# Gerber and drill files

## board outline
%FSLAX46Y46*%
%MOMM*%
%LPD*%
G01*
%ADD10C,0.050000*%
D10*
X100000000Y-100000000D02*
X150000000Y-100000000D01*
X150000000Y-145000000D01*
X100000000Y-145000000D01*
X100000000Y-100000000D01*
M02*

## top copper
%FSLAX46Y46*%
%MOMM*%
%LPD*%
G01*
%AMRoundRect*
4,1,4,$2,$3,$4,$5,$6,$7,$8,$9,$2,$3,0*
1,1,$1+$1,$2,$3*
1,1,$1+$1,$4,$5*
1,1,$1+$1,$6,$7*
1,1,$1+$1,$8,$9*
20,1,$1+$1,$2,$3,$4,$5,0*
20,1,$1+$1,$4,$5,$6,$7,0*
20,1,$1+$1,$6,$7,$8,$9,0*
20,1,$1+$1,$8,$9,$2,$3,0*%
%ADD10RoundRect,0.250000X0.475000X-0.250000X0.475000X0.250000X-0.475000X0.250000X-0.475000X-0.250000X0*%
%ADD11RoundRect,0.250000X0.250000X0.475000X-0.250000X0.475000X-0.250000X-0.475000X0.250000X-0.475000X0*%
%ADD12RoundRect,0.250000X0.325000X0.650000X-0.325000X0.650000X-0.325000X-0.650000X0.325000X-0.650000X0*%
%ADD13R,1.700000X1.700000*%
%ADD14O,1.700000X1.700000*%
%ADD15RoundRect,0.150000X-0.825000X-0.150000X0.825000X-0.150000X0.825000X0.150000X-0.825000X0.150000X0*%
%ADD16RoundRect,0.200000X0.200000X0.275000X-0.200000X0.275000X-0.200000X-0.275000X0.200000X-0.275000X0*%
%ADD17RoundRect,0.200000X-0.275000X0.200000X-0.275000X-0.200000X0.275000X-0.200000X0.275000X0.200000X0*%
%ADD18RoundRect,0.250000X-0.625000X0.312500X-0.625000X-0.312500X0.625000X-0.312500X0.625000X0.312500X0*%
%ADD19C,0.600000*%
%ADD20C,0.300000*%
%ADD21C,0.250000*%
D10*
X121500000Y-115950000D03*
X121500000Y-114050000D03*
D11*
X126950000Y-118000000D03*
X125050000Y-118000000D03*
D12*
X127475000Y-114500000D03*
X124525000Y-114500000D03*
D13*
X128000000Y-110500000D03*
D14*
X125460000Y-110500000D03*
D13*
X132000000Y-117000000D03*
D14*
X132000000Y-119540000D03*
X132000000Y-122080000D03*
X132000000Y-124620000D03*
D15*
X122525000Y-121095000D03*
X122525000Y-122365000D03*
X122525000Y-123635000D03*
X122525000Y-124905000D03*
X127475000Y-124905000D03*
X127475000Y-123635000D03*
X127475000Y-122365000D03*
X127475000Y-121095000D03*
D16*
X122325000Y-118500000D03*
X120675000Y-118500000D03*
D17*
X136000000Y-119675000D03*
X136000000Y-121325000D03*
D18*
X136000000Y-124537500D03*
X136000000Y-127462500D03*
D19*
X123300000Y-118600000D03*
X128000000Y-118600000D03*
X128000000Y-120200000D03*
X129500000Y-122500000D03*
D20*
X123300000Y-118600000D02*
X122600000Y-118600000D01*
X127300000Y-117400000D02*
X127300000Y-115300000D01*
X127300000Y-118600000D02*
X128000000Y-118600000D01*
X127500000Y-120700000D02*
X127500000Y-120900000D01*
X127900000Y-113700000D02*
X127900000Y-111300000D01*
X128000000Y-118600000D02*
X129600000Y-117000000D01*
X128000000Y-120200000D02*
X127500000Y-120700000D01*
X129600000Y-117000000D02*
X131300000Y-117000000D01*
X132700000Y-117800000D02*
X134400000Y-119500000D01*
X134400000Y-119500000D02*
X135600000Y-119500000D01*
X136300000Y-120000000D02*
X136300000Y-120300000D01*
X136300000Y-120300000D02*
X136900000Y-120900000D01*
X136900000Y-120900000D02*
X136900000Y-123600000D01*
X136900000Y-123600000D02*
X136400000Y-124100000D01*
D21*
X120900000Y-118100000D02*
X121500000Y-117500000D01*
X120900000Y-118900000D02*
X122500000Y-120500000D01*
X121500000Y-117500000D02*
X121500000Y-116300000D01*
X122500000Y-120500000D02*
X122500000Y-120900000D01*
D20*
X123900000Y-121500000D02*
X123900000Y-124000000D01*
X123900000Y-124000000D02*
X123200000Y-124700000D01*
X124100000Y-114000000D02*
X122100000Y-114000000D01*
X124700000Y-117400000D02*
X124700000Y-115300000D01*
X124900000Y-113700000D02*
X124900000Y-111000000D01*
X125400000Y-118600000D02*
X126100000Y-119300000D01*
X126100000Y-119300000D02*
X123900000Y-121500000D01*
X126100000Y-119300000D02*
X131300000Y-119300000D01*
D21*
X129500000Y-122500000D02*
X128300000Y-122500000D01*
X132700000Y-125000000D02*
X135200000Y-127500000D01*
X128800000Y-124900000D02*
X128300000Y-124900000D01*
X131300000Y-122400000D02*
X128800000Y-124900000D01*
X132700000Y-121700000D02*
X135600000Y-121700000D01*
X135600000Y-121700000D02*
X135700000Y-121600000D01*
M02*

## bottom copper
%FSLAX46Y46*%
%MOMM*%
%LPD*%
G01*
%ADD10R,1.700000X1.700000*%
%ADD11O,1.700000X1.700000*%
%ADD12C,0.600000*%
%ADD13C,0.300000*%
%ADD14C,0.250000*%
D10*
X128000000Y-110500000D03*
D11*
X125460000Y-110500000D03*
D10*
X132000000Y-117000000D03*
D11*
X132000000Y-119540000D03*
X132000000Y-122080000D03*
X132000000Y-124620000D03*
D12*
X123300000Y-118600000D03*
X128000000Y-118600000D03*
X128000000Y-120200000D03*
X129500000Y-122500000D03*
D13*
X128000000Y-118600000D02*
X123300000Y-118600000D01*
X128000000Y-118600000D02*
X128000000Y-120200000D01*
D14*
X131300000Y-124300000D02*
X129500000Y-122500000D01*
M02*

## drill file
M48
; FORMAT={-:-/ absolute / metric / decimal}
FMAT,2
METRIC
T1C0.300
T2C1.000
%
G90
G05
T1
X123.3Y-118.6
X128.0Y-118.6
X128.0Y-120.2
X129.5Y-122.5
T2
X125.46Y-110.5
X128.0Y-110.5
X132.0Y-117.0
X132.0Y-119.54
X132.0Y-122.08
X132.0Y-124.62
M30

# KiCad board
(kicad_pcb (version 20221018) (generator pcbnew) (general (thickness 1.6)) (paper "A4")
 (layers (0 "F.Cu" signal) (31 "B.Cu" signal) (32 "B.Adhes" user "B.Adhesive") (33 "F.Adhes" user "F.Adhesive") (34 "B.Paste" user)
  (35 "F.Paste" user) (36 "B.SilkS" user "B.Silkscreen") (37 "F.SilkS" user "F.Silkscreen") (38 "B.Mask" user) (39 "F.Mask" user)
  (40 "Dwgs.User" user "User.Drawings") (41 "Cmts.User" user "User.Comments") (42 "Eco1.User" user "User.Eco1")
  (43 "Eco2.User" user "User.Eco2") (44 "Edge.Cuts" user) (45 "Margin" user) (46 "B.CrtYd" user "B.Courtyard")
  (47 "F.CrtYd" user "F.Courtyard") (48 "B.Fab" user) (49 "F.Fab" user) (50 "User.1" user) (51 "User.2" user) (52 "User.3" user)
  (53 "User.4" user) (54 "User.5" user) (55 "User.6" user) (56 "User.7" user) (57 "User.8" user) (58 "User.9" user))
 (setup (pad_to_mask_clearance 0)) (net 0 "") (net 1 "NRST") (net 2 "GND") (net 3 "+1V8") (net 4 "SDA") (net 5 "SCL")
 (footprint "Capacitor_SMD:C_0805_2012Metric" (layer "F.Cu") (at 121.5 115 90)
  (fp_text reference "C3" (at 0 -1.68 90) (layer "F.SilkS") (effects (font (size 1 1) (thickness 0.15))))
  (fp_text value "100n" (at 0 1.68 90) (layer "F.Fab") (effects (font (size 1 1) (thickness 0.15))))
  (pad "1" smd roundrect (at -0.95 0 90) (size 1 1.45) (layers "F.Cu" "F.Paste" "F.Mask") (roundrect_rratio 0.25) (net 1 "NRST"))
  (pad "2" smd roundrect (at 0.95 0 90) (size 1 1.45) (layers "F.Cu" "F.Paste" "F.Mask") (roundrect_rratio 0.25) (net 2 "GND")))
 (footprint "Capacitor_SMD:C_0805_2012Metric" (layer "F.Cu") (at 126 118 180)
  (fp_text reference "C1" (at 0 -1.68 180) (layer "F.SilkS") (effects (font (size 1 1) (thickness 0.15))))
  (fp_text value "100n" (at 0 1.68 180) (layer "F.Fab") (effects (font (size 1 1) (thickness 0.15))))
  (pad "1" smd roundrect (at -0.95 0 180) (size 1 1.45) (layers "F.Cu" "F.Paste" "F.Mask") (roundrect_rratio 0.25) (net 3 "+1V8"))
  (pad "2" smd roundrect (at 0.95 0 180) (size 1 1.45) (layers "F.Cu" "F.Paste" "F.Mask") (roundrect_rratio 0.25) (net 2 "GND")))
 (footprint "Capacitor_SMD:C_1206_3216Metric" (layer "F.Cu") (at 126 114.5 180)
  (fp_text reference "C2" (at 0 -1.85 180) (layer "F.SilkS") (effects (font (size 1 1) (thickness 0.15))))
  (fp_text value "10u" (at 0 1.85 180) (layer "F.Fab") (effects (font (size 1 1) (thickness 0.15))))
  (pad "1" smd roundrect (at -1.475 0 180) (size 1.15 1.8) (layers "F.Cu" "F.Paste" "F.Mask") (roundrect_rratio 0.217391) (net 3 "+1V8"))
  (pad "2" smd roundrect (at 1.475 0 180) (size 1.15 1.8) (layers "F.Cu" "F.Paste" "F.Mask") (roundrect_rratio 0.217391) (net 2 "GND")))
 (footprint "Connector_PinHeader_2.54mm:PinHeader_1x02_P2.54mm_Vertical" (layer "F.Cu") (at 128 110.5 -90)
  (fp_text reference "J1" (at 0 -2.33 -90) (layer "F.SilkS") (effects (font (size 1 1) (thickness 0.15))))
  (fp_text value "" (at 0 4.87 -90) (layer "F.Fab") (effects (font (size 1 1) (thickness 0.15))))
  (pad "1" thru_hole rect (at 0 0 270) (size 1.7 1.7) (drill 1) (layers "*.Cu" "*.Mask") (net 3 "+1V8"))
  (pad "2" thru_hole oval (at 0 2.54 270) (size 1.7 1.7) (drill 1) (layers "*.Cu" "*.Mask") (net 2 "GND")))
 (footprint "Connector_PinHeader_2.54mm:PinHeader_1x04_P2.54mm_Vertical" (layer "F.Cu") (at 132 117)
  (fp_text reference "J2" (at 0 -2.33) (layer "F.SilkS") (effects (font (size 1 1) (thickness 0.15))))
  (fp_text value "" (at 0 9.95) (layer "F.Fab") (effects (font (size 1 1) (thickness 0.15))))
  (pad "1" thru_hole rect (at 0 0) (size 1.7 1.7) (drill 1) (layers "*.Cu" "*.Mask") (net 3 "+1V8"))
  (pad "2" thru_hole oval (at 0 2.54) (size 1.7 1.7) (drill 1) (layers "*.Cu" "*.Mask") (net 2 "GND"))
  (pad "3" thru_hole oval (at 0 5.08) (size 1.7 1.7) (drill 1) (layers "*.Cu" "*.Mask") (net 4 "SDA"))
  (pad "4" thru_hole oval (at 0 7.62) (size 1.7 1.7) (drill 1) (layers "*.Cu" "*.Mask") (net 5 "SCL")))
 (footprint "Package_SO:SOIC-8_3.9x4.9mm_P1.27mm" (layer "F.Cu") (at 125 123)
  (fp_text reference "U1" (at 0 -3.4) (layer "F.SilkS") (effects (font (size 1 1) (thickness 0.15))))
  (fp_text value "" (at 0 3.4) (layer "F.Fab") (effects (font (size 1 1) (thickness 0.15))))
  (pad "1" smd roundrect (at -2.475 -1.905) (size 1.95 0.6) (layers "F.Cu" "F.Paste" "F.Mask") (roundrect_rratio 0.25) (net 1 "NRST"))
  (pad "2" smd roundrect (at -2.475 -0.635) (size 1.95 0.6) (layers "F.Cu" "F.Paste" "F.Mask") (roundrect_rratio 0.25))
  (pad "3" smd roundrect (at -2.475 0.635) (size 1.95 0.6) (layers "F.Cu" "F.Paste" "F.Mask") (roundrect_rratio 0.25))
  (pad "4" smd roundrect (at -2.475 1.905) (size 1.95 0.6) (layers "F.Cu" "F.Paste" "F.Mask") (roundrect_rratio 0.25) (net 2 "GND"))
  (pad "5" smd roundrect (at 2.475 1.905) (size 1.95 0.6) (layers "F.Cu" "F.Paste" "F.Mask") (roundrect_rratio 0.25) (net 4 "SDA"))
  (pad "6" smd roundrect (at 2.475 0.635) (size 1.95 0.6) (layers "F.Cu" "F.Paste" "F.Mask") (roundrect_rratio 0.25))
  (pad "7" smd roundrect (at 2.475 -0.635) (size 1.95 0.6) (layers "F.Cu" "F.Paste" "F.Mask") (roundrect_rratio 0.25) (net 5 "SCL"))
  (pad "8" smd roundrect (at 2.475 -1.905) (size 1.95 0.6) (layers "F.Cu" "F.Paste" "F.Mask") (roundrect_rratio 0.25) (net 3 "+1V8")))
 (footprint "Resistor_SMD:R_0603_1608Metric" (layer "F.Cu") (at 121.5 118.5 180)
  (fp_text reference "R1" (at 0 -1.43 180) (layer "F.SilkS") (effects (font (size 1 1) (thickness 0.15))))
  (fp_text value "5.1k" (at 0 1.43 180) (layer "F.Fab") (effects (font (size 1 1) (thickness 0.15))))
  (pad "1" smd roundrect (at -0.825 0 180) (size 0.8 0.95) (layers "F.Cu" "F.Paste" "F.Mask") (roundrect_rratio 0.25) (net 3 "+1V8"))
  (pad "2" smd roundrect (at 0.825 0 180) (size 0.8 0.95) (layers "F.Cu" "F.Paste" "F.Mask") (roundrect_rratio 0.25) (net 1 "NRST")))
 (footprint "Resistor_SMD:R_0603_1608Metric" (layer "F.Cu") (at 136 120.5 -90)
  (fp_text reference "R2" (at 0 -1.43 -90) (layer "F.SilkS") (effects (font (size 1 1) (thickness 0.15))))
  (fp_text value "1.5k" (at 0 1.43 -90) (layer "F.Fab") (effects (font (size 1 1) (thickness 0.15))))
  (pad "1" smd roundrect (at -0.825 0 270) (size 0.8 0.95) (layers "F.Cu" "F.Paste" "F.Mask") (roundrect_rratio 0.25) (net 3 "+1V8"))
  (pad "2" smd roundrect (at 0.825 0 270) (size 0.8 0.95) (layers "F.Cu" "F.Paste" "F.Mask") (roundrect_rratio 0.25) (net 4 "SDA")))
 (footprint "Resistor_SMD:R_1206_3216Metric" (layer "F.Cu") (at 136 126 -90)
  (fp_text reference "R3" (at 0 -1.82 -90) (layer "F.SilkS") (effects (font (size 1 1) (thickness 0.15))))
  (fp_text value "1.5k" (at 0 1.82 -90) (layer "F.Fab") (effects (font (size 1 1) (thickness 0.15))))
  (pad "1" smd roundrect (at -1.4625 0 270) (size 1.125 1.75) (layers "F.Cu" "F.Paste" "F.Mask") (roundrect_rratio 0.222222) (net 3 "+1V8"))
  (pad "2" smd roundrect (at 1.4625 0 270) (size 1.125 1.75) (layers "F.Cu" "F.Paste" "F.Mask") (roundrect_rratio 0.222222) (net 5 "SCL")))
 (gr_rect (start 100 100) (end 150 145) (stroke (width 0.05) (type default)) (fill none) (layer "Edge.Cuts"))
 (segment (start 123.3 118.6) (end 122.6 118.6) (width 0.3) (layer "F.Cu") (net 3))
 (segment (start 127.3 117.4) (end 127.3 115.3) (width 0.3) (layer "F.Cu") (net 3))
 (segment (start 127.3 118.6) (end 128 118.6) (width 0.3) (layer "F.Cu") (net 3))
 (segment (start 127.5 120.7) (end 127.5 120.9) (width 0.3) (layer "F.Cu") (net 3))
 (segment (start 127.9 113.7) (end 127.9 111.3) (width 0.3) (layer "F.Cu") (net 3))
 (segment (start 128 118.6) (end 129.6 117) (width 0.3) (layer "F.Cu") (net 3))
 (segment (start 128 120.2) (end 127.5 120.7) (width 0.3) (layer "F.Cu") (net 3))
 (segment (start 129.6 117) (end 131.3 117) (width 0.3) (layer "F.Cu") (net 3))
 (segment (start 132.7 117.8) (end 134.4 119.5) (width 0.3) (layer "F.Cu") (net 3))
 (segment (start 134.4 119.5) (end 135.6 119.5) (width 0.3) (layer "F.Cu") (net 3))
 (segment (start 136.3 120) (end 136.3 120.3) (width 0.3) (layer "F.Cu") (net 3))
 (segment (start 136.3 120.3) (end 136.9 120.9) (width 0.3) (layer "F.Cu") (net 3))
 (segment (start 136.9 120.9) (end 136.9 123.6) (width 0.3) (layer "F.Cu") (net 3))
 (segment (start 136.9 123.6) (end 136.4 124.1) (width 0.3) (layer "F.Cu") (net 3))
 (via (at 123.3 118.6) (size 0.6) (drill 0.3) (layers "F.Cu" "B.Cu") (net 3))
 (via (at 128 118.6) (size 0.6) (drill 0.3) (layers "F.Cu" "B.Cu") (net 3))
 (via (at 128 120.2) (size 0.6) (drill 0.3) (layers "F.Cu" "B.Cu") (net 3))
 (segment (start 120.9 118.1) (end 121.5 117.5) (width 0.25) (layer "F.Cu") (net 1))
 (segment (start 120.9 118.9) (end 122.5 120.5) (width 0.25) (layer "F.Cu") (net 1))
 (segment (start 121.5 117.5) (end 121.5 116.3) (width 0.25) (layer "F.Cu") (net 1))
 (segment (start 122.5 120.5) (end 122.5 120.9) (width 0.25) (layer "F.Cu") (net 1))
 (segment (start 123.9 121.5) (end 123.9 124) (width 0.3) (layer "F.Cu") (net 2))
 (segment (start 123.9 124) (end 123.2 124.7) (width 0.3) (layer "F.Cu") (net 2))
 (segment (start 124.1 114) (end 122.1 114) (width 0.3) (layer "F.Cu") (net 2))
 (segment (start 124.7 117.4) (end 124.7 115.3) (width 0.3) (layer "F.Cu") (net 2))
 (segment (start 124.9 113.7) (end 124.9 111) (width 0.3) (layer "F.Cu") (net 2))
 (segment (start 125.4 118.6) (end 126.1 119.3) (width 0.3) (layer "F.Cu") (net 2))
 (segment (start 126.1 119.3) (end 123.9 121.5) (width 0.3) (layer "F.Cu") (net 2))
 (segment (start 126.1 119.3) (end 131.3 119.3) (width 0.3) (layer "F.Cu") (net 2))
 (segment (start 128 118.6) (end 123.3 118.6) (width 0.3) (layer "B.Cu") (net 3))
 (segment (start 128 118.6) (end 128 120.2) (width 0.3) (layer "B.Cu") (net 3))
 (segment (start 129.5 122.5) (end 128.3 122.5) (width 0.25) (layer "F.Cu") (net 5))
 (segment (start 132.7 125) (end 135.2 127.5) (width 0.25) (layer "F.Cu") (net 5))
 (via (at 129.5 122.5) (size 0.6) (drill 0.3) (layers "F.Cu" "B.Cu") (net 5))
 (segment (start 128.8 124.9) (end 128.3 124.9) (width 0.25) (layer "F.Cu") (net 4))
 (segment (start 131.3 122.4) (end 128.8 124.9) (width 0.25) (layer "F.Cu") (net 4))
 (segment (start 131.3 124.3) (end 129.5 122.5) (width 0.25) (layer "B.Cu") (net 5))
 (segment (start 132.7 121.7) (end 135.6 121.7) (width 0.25) (layer "F.Cu") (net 4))
 (segment (start 135.6 121.7) (end 135.7 121.6) (width 0.25) (layer "F.Cu") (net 4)))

